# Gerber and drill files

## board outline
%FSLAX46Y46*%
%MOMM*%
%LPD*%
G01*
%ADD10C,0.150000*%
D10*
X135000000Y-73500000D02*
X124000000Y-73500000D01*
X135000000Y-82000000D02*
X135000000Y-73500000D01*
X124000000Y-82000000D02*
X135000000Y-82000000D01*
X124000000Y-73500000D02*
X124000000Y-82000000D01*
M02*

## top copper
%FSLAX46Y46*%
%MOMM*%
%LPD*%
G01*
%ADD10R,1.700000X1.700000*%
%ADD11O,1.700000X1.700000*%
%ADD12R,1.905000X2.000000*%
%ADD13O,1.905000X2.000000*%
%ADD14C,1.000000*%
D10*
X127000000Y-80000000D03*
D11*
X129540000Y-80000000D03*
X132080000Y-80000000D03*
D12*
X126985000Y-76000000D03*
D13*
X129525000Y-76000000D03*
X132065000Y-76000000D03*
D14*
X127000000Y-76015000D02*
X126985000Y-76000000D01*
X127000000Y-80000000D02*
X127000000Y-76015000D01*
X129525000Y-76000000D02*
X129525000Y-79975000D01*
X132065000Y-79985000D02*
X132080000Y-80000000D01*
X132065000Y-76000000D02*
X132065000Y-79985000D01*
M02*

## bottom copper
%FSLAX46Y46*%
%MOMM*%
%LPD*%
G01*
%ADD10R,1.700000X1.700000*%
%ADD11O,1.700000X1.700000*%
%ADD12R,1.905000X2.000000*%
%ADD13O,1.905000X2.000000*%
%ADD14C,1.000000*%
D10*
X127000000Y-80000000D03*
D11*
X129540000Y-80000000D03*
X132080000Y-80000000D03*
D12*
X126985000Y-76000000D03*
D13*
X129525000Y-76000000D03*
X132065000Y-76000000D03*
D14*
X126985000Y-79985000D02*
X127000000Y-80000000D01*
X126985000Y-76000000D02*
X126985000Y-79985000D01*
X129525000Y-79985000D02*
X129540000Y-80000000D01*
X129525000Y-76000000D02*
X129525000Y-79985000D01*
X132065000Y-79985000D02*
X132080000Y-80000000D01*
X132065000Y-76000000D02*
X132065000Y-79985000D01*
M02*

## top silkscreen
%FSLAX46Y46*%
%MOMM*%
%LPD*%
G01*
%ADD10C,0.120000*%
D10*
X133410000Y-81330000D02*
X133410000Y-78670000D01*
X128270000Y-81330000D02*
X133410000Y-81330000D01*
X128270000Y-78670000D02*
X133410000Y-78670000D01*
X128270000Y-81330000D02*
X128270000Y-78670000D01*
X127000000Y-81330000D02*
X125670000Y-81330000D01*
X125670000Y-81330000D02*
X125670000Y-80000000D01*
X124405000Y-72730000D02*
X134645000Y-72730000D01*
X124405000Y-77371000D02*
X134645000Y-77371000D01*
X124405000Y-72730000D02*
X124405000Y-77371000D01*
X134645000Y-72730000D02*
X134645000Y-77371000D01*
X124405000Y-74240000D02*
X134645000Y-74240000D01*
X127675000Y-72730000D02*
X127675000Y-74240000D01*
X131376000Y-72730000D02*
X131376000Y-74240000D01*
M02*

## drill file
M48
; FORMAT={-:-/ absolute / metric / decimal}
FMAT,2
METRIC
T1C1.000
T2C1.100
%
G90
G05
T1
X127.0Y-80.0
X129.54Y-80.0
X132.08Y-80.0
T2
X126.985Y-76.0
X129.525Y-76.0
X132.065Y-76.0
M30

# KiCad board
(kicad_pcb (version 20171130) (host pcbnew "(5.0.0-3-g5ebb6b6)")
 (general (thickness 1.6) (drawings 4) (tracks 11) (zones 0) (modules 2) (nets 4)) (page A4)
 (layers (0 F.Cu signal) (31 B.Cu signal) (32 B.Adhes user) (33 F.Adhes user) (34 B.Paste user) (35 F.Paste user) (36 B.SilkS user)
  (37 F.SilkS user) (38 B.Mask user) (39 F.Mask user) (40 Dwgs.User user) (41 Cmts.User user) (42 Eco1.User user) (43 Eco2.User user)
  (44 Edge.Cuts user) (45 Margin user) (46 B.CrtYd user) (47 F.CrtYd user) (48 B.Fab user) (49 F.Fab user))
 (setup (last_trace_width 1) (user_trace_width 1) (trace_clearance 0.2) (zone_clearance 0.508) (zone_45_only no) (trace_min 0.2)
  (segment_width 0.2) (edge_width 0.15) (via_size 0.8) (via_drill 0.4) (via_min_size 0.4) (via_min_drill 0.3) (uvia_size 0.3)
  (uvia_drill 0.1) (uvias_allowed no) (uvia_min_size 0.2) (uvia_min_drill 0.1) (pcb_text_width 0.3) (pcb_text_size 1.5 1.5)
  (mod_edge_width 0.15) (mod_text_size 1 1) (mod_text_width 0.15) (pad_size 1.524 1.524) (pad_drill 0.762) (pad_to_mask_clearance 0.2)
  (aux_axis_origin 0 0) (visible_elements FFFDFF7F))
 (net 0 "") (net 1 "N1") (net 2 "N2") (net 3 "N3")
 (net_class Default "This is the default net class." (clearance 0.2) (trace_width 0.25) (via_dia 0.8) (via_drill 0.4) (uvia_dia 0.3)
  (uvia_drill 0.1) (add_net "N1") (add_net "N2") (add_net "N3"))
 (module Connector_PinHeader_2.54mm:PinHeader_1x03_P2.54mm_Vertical (layer F.Cu) (at 127 80 90)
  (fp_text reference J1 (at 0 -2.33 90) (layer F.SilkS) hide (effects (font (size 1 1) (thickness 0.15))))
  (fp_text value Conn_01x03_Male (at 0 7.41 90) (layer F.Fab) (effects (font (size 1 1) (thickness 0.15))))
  (fp_line (start -1.33 6.41) (end 1.33 6.41) (layer F.SilkS) (width 0.12))
  (fp_line (start -1.33 1.27) (end -1.33 6.41) (layer F.SilkS) (width 0.12))
  (fp_line (start 1.33 1.27) (end 1.33 6.41) (layer F.SilkS) (width 0.12))
  (fp_line (start -1.33 1.27) (end 1.33 1.27) (layer F.SilkS) (width 0.12))
  (fp_line (start -1.33 0) (end -1.33 -1.33) (layer F.SilkS) (width 0.12))
  (fp_line (start -1.33 -1.33) (end 0 -1.33) (layer F.SilkS) (width 0.12))
  (pad 1 thru_hole rect (at 0 0 90) (size 1.7 1.7) (drill 1) (layers *.Cu *.Mask) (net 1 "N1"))
  (pad 2 thru_hole oval (at 0 2.54 90) (size 1.7 1.7) (drill 1) (layers *.Cu *.Mask) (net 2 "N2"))
  (pad 3 thru_hole oval (at 0 5.08 90) (size 1.7 1.7) (drill 1) (layers *.Cu *.Mask) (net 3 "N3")))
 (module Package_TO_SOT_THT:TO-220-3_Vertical (layer F.Cu) (at 126.985 76)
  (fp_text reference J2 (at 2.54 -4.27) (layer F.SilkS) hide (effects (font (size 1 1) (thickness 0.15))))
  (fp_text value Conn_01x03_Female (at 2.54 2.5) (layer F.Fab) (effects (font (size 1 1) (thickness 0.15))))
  (fp_line (start -2.58 -3.27) (end 7.66 -3.27) (layer F.SilkS) (width 0.12))
  (fp_line (start -2.58 1.371) (end 7.66 1.371) (layer F.SilkS) (width 0.12))
  (fp_line (start -2.58 -3.27) (end -2.58 1.371) (layer F.SilkS) (width 0.12))
  (fp_line (start 7.66 -3.27) (end 7.66 1.371) (layer F.SilkS) (width 0.12))
  (fp_line (start -2.58 -1.76) (end 7.66 -1.76) (layer F.SilkS) (width 0.12))
  (fp_line (start 0.69 -3.27) (end 0.69 -1.76) (layer F.SilkS) (width 0.12))
  (fp_line (start 4.391 -3.27) (end 4.391 -1.76) (layer F.SilkS) (width 0.12))
  (pad 1 thru_hole rect (at 0 0) (size 1.905 2) (drill 1.1) (layers *.Cu *.Mask) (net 1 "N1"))
  (pad 2 thru_hole oval (at 2.54 0) (size 1.905 2) (drill 1.1) (layers *.Cu *.Mask) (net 2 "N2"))
  (pad 3 thru_hole oval (at 5.08 0) (size 1.905 2) (drill 1.1) (layers *.Cu *.Mask) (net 3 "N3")))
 (gr_line (start 135 73.5) (end 124 73.5) (layer Edge.Cuts) (width 0.15))
 (gr_line (start 135 82) (end 135 73.5) (layer Edge.Cuts) (width 0.15))
 (gr_line (start 124 82) (end 135 82) (layer Edge.Cuts) (width 0.15))
 (gr_line (start 124 73.5) (end 124 82) (layer Edge.Cuts) (width 0.15))
 (segment (start 127 76.015) (end 126.985 76) (width 1) (layer F.Cu) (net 1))
 (segment (start 127 80) (end 127 76.015) (width 1) (layer F.Cu) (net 1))
 (segment (start 126.985 79.985) (end 127 80) (width 1) (layer B.Cu) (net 1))
 (segment (start 126.985 76) (end 126.985 79.985) (width 1) (layer B.Cu) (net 1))
 (segment (start 129.525 76) (end 129.525 79.975) (width 1) (layer F.Cu) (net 2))
 (segment (start 129.525 79.985) (end 129.54 80) (width 1) (layer B.Cu) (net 2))
 (segment (start 129.525 76) (end 129.525 79.985) (width 1) (layer B.Cu) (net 2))
 (segment (start 132.065 79.985) (end 132.08 80) (width 1) (layer F.Cu) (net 3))
 (segment (start 132.065 76) (end 132.065 79.985) (width 1) (layer F.Cu) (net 3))
 (segment (start 132.065 79.985) (end 132.08 80) (width 1) (layer B.Cu) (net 3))
 (segment (start 132.065 76) (end 132.065 79.985) (width 1) (layer B.Cu) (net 3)))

